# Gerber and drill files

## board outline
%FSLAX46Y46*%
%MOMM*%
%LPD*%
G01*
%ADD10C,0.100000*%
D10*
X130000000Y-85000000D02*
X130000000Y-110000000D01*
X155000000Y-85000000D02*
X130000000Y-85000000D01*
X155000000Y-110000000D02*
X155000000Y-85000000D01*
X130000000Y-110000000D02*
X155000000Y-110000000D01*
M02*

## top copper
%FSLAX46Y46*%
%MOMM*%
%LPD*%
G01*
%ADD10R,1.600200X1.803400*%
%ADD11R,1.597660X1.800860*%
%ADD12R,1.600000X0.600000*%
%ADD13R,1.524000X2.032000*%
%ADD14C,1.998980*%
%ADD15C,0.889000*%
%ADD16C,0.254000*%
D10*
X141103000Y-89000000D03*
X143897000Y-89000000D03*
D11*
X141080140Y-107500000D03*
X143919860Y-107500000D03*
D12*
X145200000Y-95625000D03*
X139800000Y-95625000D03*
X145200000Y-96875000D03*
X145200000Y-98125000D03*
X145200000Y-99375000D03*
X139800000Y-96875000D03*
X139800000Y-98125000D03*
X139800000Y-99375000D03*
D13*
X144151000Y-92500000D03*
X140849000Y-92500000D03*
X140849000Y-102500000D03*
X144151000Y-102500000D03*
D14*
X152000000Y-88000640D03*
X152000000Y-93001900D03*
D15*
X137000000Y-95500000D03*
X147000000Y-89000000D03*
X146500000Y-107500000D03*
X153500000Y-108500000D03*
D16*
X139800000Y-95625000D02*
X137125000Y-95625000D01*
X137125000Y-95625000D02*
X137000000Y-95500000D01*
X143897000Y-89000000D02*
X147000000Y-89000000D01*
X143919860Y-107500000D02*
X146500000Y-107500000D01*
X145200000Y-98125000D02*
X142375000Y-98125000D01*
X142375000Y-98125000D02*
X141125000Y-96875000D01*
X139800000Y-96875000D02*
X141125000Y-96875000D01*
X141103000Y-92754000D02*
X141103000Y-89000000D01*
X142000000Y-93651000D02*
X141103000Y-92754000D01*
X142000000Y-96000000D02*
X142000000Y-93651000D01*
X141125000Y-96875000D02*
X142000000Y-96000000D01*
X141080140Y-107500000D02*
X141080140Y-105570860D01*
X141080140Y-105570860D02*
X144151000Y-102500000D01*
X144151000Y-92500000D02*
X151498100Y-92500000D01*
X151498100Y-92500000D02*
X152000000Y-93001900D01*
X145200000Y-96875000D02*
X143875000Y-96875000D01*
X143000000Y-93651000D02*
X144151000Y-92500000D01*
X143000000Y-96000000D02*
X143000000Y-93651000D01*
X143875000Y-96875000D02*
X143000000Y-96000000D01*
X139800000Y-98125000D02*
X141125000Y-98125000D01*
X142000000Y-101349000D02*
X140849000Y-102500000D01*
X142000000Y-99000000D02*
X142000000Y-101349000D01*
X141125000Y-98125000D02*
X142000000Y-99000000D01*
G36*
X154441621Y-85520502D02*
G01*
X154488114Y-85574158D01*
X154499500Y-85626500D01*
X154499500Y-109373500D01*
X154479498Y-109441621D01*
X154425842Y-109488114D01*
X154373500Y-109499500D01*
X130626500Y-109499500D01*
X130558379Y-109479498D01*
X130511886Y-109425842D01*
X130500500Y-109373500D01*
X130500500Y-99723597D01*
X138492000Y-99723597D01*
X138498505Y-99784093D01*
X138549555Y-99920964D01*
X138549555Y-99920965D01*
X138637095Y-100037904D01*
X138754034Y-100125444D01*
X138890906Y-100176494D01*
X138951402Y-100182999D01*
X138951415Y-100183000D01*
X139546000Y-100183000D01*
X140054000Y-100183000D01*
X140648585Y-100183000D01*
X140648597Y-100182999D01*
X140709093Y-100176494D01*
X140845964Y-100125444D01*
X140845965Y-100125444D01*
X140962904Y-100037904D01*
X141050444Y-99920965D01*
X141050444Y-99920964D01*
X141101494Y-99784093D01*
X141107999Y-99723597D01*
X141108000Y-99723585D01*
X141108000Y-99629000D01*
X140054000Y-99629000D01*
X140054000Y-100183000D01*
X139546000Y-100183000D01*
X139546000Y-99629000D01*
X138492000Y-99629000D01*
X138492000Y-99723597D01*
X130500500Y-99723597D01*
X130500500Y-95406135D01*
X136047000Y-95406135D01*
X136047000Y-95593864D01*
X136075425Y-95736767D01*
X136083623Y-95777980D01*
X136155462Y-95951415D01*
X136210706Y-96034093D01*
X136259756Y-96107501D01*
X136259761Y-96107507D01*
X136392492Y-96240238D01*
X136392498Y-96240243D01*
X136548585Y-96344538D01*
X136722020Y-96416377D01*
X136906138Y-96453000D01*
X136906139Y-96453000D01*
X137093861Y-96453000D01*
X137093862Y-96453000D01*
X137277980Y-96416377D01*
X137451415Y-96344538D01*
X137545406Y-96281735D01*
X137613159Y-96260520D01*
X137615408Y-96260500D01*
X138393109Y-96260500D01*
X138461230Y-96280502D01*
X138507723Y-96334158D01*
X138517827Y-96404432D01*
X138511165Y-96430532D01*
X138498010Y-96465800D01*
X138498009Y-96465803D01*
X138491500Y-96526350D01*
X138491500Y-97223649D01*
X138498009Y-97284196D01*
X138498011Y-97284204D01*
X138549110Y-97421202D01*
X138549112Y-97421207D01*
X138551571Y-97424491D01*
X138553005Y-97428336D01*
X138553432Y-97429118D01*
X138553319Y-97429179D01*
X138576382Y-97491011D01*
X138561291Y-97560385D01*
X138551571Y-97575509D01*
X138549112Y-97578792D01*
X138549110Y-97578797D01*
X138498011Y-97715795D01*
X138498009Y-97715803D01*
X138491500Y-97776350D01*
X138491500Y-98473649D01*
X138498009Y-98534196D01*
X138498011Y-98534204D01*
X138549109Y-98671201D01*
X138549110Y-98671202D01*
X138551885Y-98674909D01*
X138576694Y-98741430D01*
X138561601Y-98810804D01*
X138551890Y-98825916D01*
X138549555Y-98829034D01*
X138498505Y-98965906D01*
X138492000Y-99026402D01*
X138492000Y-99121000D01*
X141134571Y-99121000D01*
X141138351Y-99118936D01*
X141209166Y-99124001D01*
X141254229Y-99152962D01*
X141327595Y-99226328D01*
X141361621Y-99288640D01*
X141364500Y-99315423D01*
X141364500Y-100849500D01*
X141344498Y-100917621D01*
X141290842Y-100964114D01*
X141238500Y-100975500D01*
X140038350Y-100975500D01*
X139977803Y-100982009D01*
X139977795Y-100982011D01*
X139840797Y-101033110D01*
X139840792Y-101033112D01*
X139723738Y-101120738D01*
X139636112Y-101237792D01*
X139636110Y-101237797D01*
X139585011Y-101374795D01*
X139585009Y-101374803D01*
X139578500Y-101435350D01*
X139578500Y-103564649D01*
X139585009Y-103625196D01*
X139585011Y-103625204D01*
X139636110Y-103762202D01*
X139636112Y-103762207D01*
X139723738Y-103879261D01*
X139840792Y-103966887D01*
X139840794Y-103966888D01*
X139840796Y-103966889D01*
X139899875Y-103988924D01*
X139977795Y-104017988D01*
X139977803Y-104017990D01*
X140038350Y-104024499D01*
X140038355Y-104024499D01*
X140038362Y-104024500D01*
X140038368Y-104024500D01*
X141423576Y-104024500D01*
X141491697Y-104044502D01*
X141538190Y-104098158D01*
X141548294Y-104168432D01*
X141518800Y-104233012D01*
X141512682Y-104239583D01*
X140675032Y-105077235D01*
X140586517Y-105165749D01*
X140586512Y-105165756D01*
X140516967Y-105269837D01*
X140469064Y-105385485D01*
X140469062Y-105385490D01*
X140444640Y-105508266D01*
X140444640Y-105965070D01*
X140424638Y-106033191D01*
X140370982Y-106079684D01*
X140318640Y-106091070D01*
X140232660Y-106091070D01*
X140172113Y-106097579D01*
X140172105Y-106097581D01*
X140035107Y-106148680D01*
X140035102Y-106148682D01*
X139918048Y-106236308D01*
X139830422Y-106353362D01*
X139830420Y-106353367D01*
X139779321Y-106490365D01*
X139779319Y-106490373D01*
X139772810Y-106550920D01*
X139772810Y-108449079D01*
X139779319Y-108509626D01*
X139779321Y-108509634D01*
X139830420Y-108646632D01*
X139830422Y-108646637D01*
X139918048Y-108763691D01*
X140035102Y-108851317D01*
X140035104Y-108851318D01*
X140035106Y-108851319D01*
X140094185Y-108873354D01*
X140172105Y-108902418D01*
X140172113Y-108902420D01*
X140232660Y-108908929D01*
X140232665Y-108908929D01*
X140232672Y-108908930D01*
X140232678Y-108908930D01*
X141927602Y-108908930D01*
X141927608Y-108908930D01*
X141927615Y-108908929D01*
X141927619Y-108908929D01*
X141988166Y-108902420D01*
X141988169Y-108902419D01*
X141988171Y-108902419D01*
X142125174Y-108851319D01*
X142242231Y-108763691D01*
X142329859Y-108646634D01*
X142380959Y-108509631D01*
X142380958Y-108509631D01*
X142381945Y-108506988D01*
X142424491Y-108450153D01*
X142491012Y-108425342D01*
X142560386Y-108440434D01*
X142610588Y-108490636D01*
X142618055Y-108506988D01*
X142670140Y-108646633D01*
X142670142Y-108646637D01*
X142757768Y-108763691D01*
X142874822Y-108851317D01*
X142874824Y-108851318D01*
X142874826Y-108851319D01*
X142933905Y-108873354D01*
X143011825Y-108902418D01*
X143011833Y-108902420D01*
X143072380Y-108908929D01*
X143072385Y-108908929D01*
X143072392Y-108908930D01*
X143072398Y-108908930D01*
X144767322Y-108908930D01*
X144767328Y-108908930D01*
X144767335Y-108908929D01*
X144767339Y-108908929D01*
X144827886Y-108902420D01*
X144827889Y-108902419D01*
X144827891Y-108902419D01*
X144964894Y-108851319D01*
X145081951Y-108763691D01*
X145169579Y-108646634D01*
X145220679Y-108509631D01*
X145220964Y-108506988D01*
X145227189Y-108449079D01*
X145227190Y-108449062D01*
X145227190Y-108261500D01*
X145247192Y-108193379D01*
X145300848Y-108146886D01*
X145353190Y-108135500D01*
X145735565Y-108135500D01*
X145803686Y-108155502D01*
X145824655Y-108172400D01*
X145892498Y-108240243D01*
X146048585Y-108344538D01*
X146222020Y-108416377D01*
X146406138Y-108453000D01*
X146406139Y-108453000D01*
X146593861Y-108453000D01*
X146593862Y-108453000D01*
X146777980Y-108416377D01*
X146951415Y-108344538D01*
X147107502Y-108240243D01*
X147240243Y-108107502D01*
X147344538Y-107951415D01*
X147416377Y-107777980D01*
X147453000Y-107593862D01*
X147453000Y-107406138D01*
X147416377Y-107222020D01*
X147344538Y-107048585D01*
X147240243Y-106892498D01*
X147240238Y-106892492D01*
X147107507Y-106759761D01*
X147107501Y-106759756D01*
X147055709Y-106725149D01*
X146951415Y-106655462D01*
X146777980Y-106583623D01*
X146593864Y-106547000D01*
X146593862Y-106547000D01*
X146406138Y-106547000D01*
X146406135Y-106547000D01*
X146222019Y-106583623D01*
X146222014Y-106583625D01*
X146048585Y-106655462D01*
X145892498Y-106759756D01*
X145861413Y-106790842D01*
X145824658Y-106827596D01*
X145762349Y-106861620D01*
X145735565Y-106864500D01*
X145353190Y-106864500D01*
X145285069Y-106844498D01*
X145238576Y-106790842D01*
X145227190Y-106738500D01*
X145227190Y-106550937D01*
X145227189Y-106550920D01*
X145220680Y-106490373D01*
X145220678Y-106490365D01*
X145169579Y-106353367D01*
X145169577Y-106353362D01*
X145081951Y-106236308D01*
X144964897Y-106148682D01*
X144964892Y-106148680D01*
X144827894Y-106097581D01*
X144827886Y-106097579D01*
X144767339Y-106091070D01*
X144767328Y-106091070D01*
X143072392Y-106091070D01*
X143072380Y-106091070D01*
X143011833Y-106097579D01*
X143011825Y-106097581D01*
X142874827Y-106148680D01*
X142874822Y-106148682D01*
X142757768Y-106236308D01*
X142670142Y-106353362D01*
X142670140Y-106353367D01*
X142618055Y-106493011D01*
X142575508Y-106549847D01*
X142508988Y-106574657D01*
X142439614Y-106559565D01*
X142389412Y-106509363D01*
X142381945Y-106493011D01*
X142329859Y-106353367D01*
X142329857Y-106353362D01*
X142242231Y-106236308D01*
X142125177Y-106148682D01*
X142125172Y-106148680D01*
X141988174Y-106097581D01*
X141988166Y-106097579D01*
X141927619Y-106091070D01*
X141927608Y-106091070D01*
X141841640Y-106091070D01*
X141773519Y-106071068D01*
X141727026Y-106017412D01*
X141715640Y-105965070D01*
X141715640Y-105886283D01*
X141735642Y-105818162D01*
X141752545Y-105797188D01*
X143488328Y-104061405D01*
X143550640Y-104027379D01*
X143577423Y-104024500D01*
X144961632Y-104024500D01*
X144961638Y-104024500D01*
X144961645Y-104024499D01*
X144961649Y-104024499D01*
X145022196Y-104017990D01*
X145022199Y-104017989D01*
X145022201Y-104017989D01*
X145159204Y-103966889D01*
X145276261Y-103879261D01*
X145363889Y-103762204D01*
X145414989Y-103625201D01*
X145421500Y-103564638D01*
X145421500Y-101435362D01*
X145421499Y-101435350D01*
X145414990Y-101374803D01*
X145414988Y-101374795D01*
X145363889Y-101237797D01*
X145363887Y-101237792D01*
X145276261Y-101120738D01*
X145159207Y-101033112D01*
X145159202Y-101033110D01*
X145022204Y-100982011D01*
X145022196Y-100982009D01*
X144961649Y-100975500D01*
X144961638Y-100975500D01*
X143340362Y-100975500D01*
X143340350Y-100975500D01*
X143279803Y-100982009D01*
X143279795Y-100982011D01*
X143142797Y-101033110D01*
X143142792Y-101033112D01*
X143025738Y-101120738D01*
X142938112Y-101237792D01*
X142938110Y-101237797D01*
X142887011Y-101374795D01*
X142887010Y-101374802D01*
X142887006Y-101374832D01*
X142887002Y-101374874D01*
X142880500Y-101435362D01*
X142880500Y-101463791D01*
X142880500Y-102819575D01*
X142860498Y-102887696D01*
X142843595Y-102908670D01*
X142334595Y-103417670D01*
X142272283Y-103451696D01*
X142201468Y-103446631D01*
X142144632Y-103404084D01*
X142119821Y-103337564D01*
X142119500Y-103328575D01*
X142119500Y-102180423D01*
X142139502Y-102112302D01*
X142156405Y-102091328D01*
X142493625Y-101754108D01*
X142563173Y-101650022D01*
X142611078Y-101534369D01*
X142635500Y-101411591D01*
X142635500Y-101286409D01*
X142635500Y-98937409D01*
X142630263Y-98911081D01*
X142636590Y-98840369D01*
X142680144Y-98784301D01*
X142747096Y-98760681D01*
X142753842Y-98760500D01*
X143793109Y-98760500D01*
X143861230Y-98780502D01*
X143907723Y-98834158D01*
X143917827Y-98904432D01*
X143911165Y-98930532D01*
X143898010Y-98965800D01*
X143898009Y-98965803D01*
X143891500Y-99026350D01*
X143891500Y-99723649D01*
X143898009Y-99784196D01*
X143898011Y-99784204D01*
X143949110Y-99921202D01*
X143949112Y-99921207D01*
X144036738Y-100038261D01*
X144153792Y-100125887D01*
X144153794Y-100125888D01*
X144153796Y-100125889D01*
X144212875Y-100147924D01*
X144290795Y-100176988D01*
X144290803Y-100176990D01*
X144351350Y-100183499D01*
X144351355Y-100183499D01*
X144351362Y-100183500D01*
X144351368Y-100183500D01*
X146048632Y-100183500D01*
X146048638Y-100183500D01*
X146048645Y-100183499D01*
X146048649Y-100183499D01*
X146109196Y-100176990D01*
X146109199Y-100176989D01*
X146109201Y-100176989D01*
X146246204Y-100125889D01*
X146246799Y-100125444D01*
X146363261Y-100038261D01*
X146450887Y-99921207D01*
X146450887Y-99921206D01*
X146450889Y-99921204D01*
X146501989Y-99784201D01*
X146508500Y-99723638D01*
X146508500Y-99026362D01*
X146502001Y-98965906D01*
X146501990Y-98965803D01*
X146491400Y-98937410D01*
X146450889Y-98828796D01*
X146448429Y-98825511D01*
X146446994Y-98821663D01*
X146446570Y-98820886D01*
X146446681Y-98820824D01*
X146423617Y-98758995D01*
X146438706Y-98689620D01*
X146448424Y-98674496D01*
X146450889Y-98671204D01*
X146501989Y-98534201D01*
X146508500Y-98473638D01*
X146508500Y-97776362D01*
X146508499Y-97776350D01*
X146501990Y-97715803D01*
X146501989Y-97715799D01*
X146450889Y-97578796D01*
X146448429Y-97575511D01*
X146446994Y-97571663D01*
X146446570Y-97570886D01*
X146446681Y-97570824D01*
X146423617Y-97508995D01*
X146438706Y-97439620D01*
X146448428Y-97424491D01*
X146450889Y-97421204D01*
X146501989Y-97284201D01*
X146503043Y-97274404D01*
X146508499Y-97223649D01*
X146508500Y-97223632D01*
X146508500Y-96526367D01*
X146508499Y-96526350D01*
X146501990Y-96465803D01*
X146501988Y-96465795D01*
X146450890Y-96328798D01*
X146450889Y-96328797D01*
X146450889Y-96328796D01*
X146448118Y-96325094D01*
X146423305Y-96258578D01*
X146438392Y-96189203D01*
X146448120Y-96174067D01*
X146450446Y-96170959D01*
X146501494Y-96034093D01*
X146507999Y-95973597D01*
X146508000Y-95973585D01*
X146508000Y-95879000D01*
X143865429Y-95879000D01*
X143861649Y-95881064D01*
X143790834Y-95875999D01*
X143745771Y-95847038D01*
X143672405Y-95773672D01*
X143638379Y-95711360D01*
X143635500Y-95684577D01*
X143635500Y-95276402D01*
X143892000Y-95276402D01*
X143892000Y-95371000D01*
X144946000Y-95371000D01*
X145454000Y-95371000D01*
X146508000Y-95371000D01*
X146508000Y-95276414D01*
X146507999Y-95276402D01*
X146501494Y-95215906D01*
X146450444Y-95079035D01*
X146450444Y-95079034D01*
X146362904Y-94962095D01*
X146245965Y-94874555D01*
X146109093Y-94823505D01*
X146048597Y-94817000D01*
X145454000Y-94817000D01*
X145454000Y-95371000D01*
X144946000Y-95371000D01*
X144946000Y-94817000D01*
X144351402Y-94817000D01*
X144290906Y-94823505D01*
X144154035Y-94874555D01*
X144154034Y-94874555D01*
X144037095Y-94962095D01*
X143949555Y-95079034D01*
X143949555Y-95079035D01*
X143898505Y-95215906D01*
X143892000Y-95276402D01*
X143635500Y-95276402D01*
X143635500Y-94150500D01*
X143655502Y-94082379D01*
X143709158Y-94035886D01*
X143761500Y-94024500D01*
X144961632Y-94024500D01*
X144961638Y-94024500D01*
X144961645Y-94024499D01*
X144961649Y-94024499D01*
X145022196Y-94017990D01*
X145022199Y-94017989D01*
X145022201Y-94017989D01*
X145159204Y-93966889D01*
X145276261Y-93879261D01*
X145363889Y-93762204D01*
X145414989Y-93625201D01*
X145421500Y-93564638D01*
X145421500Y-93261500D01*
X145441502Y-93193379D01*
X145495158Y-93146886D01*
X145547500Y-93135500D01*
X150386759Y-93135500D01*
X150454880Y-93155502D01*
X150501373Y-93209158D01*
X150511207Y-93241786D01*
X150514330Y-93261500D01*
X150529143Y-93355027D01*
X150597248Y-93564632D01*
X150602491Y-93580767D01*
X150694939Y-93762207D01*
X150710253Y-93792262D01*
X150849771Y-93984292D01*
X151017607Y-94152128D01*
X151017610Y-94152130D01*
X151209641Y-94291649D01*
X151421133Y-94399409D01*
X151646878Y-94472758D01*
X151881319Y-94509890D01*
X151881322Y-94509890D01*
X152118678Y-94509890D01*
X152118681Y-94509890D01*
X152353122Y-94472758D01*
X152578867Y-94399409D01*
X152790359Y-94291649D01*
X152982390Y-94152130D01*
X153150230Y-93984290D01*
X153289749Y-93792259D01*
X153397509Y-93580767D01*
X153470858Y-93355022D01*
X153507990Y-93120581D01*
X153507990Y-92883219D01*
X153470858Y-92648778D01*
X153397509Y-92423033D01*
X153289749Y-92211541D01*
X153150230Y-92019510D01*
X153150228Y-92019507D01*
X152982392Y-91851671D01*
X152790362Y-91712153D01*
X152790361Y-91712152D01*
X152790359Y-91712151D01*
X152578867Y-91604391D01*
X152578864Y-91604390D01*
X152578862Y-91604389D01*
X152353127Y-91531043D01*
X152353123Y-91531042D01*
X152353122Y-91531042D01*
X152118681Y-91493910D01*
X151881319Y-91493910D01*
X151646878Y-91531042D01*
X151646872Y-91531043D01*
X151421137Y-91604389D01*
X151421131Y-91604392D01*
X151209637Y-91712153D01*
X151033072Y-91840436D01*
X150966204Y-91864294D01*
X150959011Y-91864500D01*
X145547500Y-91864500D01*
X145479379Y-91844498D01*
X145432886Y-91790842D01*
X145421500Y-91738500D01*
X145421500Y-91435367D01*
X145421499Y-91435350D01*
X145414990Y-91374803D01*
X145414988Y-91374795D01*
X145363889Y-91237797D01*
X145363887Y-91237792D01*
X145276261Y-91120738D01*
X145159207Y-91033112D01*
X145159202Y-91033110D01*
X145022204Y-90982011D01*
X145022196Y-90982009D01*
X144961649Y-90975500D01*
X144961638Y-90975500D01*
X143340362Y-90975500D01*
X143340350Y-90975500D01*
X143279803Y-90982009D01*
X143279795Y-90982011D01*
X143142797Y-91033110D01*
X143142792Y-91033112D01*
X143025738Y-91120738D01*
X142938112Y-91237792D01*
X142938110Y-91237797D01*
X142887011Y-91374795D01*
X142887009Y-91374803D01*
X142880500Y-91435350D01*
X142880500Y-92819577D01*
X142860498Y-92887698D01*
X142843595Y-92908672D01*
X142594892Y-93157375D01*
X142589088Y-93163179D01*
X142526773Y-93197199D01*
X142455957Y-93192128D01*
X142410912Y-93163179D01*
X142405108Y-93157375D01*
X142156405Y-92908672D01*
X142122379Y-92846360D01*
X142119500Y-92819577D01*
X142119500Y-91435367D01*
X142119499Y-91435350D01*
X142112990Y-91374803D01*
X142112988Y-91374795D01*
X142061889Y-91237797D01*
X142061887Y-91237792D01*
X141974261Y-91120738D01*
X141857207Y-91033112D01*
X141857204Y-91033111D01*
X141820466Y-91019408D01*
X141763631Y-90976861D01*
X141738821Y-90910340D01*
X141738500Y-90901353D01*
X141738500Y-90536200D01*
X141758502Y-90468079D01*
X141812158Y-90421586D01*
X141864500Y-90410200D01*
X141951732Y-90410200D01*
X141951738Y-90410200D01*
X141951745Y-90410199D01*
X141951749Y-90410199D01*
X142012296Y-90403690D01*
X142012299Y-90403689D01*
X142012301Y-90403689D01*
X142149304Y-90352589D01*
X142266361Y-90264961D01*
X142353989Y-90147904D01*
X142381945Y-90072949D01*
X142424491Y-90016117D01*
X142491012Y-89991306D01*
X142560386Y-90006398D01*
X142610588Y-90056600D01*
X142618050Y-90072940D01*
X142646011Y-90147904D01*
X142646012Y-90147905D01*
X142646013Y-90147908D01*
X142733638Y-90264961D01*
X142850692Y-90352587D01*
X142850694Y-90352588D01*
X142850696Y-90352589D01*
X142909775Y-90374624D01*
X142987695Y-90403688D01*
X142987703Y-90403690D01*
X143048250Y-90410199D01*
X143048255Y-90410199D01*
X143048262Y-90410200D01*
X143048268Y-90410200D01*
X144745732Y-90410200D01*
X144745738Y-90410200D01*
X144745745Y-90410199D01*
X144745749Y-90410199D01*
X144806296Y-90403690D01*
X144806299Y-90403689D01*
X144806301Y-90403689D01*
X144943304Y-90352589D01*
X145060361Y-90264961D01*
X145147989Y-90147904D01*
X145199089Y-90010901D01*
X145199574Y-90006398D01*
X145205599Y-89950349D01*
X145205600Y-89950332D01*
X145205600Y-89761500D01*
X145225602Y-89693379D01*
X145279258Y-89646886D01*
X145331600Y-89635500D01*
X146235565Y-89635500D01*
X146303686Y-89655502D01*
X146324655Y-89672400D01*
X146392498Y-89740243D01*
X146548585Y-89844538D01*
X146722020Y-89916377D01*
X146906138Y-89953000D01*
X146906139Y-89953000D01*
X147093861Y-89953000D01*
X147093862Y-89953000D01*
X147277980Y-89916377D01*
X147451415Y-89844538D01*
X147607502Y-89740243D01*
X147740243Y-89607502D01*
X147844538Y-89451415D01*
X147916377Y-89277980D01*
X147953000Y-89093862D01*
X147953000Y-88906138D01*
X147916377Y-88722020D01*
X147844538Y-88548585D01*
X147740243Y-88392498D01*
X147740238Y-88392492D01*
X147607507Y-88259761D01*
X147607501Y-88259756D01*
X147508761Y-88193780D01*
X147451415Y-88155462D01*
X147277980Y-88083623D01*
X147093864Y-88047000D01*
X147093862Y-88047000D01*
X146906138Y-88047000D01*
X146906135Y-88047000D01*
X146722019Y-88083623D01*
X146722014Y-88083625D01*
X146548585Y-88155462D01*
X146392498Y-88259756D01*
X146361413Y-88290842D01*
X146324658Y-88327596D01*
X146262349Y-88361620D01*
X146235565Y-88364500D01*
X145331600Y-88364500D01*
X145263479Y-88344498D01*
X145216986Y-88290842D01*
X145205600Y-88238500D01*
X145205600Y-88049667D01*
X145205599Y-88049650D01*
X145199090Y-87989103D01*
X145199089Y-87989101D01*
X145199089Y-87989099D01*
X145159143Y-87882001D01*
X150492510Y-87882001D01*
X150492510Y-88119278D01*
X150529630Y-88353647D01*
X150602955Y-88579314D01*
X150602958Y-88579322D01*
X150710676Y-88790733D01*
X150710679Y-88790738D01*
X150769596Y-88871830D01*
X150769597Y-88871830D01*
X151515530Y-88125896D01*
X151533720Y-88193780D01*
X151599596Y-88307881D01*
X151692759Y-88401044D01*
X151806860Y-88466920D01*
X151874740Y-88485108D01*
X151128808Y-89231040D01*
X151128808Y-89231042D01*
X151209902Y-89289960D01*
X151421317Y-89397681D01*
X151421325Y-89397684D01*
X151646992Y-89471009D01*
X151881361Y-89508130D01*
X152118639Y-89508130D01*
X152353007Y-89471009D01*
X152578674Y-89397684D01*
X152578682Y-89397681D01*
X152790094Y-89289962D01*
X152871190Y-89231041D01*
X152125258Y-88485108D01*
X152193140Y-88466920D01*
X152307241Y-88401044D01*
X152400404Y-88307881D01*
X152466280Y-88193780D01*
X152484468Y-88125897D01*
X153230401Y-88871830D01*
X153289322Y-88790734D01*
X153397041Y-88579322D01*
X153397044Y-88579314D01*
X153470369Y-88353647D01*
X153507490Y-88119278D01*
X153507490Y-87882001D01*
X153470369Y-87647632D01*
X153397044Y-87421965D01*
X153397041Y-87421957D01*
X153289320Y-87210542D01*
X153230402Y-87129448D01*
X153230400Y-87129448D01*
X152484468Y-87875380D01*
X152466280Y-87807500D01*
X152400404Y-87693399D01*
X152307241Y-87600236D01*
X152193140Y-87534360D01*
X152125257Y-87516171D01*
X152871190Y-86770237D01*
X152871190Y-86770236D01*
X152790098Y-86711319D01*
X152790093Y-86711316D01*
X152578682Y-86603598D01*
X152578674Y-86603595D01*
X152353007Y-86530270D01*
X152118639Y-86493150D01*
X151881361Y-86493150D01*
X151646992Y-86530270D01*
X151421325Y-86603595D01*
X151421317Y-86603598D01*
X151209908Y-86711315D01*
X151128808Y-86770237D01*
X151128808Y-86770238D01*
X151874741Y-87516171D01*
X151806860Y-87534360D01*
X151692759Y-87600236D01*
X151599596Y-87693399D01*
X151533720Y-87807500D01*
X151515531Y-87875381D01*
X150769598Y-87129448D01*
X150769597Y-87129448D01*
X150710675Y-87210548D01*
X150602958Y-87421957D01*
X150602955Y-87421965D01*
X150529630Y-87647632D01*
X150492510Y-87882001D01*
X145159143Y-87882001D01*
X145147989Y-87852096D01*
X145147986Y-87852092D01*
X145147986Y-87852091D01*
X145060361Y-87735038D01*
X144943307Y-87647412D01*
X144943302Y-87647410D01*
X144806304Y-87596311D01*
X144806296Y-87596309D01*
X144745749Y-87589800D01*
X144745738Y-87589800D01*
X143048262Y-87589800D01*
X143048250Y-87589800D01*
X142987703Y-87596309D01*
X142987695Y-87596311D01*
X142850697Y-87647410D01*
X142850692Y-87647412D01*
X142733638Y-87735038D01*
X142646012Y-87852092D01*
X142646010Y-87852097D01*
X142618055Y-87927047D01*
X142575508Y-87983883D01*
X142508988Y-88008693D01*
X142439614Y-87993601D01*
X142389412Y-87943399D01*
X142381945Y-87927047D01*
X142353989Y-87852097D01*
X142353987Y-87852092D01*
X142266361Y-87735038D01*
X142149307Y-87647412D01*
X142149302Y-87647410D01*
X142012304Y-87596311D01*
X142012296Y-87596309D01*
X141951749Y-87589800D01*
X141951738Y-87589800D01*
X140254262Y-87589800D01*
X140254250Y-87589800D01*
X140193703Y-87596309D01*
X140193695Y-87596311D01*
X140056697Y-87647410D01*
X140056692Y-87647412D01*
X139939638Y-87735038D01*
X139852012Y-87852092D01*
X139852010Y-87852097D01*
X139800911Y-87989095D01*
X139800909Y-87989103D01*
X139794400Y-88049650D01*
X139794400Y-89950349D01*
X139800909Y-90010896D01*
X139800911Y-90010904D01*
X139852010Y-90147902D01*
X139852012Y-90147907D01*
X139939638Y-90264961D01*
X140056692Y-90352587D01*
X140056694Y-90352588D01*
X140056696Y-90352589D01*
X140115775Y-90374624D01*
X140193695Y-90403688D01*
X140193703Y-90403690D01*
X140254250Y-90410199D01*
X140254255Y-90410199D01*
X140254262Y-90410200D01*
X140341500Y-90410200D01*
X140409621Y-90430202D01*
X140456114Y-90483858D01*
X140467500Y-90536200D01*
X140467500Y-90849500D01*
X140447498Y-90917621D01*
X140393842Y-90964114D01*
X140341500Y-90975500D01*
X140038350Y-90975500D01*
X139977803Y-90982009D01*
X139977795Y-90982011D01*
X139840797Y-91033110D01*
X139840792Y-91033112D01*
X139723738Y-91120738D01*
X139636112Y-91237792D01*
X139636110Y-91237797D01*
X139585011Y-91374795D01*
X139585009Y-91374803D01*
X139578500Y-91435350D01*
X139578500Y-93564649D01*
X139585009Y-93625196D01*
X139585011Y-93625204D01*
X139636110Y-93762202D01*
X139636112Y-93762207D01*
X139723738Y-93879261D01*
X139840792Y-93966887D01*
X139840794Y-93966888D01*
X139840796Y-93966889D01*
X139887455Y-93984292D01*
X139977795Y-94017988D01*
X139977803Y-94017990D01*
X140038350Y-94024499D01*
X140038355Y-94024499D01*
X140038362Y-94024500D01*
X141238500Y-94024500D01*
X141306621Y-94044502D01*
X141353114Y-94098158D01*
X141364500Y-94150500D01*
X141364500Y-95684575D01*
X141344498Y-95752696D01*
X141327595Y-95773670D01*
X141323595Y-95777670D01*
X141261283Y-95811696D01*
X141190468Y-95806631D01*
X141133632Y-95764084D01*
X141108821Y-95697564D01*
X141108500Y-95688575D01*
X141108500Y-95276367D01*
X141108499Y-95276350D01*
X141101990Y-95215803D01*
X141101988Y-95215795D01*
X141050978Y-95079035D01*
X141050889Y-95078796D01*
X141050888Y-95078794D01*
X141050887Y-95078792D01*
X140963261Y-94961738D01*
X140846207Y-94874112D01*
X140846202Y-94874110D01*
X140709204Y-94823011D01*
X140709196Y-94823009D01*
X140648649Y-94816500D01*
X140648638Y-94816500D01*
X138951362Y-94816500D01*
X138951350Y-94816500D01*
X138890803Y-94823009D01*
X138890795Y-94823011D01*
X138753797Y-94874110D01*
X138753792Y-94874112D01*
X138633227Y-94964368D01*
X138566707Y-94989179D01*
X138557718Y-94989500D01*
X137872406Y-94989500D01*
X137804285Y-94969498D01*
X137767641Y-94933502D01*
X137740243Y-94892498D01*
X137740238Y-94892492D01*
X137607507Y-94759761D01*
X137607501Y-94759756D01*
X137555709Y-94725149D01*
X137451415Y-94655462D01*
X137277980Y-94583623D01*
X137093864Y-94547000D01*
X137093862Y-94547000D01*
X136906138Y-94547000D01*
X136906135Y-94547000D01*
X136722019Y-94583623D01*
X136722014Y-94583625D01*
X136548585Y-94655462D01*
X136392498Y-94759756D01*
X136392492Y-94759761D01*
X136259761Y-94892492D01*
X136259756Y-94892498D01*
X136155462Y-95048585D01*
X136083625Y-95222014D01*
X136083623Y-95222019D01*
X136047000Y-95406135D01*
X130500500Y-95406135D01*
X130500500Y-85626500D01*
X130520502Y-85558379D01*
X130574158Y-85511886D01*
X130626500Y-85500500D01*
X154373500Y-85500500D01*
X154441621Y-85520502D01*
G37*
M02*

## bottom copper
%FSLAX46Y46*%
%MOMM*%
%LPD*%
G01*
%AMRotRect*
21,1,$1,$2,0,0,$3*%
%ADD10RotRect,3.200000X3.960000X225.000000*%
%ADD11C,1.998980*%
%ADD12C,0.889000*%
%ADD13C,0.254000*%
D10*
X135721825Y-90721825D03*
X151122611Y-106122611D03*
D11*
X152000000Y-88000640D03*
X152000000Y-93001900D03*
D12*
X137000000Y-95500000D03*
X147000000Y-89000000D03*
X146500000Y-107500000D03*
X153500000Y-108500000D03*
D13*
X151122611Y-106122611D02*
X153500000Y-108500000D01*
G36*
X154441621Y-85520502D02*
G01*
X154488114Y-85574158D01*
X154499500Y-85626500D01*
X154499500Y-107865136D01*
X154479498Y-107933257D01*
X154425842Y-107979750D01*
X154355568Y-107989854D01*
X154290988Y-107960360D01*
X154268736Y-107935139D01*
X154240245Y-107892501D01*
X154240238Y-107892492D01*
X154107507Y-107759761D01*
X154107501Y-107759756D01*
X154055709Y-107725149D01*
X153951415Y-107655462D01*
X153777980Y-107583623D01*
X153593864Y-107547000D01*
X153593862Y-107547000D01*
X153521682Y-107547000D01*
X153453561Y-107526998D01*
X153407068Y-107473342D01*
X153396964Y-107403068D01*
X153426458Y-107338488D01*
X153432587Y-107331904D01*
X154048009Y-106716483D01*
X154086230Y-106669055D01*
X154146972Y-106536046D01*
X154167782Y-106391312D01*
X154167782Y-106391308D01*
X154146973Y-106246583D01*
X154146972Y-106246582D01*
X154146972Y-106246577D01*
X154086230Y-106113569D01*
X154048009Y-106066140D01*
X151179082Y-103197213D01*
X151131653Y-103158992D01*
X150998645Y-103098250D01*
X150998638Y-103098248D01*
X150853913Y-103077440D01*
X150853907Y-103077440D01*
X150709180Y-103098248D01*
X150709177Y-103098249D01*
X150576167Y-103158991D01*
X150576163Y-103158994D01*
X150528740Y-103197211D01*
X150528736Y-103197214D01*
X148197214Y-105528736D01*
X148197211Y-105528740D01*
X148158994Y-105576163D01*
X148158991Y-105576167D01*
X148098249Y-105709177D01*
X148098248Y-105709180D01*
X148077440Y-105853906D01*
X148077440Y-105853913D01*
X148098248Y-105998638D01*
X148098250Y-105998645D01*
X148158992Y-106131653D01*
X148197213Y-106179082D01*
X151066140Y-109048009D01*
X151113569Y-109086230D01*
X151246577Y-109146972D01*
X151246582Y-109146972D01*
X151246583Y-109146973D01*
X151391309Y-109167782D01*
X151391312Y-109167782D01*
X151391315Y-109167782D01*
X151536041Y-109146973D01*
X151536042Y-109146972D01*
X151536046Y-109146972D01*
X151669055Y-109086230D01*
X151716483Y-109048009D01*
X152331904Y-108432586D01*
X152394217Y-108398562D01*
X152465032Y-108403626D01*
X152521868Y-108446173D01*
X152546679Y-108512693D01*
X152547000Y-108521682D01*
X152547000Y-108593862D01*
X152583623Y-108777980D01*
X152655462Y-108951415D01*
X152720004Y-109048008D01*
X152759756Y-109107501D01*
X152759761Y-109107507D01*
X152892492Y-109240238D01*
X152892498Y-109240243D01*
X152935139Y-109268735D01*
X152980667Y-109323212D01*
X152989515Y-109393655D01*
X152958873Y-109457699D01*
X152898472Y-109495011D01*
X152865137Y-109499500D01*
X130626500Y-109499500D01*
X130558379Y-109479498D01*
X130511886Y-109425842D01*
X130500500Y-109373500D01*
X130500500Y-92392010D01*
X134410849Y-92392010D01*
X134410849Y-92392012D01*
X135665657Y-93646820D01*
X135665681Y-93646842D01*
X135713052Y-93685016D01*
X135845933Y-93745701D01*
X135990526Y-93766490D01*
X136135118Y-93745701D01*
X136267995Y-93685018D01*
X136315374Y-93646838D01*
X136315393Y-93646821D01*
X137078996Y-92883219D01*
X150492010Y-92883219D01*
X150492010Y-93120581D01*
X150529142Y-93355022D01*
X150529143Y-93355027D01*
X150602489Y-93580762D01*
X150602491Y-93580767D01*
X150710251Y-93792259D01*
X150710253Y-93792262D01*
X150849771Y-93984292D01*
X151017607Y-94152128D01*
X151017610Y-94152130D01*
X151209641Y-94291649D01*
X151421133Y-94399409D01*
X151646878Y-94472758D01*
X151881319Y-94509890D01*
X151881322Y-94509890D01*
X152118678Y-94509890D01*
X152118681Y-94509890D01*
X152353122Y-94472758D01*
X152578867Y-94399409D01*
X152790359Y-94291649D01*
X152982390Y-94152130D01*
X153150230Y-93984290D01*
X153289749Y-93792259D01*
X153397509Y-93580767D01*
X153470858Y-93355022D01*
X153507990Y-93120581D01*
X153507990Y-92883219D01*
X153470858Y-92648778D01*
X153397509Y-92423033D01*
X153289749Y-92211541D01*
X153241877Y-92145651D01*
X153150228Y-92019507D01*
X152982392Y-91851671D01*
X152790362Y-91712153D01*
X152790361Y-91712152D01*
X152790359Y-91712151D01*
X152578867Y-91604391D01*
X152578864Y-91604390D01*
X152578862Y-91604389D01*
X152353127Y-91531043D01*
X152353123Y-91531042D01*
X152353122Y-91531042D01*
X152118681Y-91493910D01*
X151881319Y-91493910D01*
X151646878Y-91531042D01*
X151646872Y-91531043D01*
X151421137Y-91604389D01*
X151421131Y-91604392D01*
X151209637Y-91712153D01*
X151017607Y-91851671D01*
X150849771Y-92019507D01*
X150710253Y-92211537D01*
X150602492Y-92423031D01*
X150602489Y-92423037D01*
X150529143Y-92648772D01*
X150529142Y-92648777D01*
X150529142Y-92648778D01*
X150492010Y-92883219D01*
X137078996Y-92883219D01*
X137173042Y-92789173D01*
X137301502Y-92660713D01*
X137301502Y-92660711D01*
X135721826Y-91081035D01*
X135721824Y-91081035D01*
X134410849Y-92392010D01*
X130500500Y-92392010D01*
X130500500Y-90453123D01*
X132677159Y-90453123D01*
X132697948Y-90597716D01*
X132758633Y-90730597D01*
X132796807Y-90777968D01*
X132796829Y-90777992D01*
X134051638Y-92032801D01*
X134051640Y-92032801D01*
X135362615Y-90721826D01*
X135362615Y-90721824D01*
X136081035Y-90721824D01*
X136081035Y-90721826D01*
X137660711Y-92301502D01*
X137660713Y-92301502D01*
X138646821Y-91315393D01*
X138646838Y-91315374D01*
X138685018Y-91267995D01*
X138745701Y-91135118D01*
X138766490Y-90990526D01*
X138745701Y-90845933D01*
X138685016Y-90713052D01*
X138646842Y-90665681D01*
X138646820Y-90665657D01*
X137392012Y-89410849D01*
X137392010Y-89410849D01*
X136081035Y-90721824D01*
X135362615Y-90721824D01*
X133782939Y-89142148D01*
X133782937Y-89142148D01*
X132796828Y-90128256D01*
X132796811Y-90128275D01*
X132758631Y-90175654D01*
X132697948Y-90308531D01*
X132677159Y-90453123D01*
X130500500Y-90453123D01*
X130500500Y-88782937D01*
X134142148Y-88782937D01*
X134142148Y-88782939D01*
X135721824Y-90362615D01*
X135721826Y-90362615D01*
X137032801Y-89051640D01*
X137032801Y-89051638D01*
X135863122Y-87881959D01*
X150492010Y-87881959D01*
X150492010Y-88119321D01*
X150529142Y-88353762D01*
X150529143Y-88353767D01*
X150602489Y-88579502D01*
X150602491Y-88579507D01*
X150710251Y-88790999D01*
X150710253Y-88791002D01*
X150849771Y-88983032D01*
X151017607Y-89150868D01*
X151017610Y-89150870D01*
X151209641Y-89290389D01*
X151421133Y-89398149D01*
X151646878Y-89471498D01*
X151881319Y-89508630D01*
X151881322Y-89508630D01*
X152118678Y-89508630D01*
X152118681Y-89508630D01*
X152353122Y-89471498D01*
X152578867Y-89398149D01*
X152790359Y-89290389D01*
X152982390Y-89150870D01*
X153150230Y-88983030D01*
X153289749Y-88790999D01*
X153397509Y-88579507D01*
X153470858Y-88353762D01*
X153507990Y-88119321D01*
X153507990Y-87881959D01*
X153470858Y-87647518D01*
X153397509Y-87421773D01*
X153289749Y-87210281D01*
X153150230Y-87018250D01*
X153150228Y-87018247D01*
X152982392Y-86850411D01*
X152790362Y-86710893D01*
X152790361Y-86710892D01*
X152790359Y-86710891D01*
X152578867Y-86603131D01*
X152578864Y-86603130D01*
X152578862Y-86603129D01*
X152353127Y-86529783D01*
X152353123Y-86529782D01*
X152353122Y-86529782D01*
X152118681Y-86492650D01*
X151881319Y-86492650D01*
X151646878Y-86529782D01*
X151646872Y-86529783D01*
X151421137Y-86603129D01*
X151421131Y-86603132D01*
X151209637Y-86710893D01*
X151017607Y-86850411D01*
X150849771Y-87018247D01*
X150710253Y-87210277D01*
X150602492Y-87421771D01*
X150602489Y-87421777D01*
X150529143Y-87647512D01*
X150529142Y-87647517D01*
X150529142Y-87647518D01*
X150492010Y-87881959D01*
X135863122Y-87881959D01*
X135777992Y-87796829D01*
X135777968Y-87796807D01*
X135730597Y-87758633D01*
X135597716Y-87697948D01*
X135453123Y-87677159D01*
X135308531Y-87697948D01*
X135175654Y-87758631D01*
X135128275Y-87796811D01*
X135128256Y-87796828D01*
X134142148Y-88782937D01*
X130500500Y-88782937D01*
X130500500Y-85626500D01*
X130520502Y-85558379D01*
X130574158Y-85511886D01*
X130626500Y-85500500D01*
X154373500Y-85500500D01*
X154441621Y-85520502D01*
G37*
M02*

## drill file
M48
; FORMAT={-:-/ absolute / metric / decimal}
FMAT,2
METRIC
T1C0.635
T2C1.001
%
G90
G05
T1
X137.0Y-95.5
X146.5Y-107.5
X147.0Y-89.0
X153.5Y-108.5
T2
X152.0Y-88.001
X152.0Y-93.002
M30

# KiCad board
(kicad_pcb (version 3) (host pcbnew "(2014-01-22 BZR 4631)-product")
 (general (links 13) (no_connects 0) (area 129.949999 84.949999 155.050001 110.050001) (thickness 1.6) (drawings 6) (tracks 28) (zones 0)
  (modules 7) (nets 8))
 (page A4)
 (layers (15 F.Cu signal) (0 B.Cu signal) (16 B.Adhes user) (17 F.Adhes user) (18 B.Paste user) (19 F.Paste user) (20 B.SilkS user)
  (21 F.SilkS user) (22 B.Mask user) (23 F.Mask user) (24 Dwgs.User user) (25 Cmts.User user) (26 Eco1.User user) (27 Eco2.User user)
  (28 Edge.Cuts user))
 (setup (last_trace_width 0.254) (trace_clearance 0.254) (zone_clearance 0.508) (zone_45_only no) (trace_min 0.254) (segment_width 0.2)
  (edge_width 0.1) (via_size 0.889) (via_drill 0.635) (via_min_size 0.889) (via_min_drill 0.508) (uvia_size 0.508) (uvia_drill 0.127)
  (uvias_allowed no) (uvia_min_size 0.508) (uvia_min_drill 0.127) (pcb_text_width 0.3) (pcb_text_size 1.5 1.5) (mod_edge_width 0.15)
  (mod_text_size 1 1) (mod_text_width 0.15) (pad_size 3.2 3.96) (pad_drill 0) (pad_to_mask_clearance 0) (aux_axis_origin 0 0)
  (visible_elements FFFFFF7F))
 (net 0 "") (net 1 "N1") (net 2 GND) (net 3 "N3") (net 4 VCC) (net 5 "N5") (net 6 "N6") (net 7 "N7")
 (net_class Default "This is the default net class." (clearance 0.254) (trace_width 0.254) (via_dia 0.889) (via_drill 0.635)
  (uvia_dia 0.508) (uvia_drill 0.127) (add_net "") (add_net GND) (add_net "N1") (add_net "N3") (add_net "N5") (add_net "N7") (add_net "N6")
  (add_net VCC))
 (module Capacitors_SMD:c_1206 (layer F.Cu) (at 142.5 89 180)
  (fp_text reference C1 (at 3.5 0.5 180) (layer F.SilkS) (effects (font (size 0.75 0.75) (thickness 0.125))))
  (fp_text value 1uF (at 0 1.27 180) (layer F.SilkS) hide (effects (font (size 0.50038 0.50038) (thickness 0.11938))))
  (pad 1 smd rect (at 1.397 0 180) (size 1.6002 1.8034) (layers F.Cu F.Paste F.Mask) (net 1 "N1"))
  (pad 2 smd rect (at -1.397 0 180) (size 1.6002 1.8034) (layers F.Cu F.Paste F.Mask) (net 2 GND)))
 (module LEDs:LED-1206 (layer F.Cu) (at 142.5 107.5)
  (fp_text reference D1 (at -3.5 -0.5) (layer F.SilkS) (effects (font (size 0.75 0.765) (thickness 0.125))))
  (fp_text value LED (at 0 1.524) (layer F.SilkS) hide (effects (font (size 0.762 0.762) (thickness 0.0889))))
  (pad 1 smd rect (at -1.41986 0) (size 1.59766 1.80086) (layers F.Cu F.Paste F.Mask) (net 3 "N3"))
  (pad 2 smd rect (at 1.41986 0) (size 1.59766 1.80086) (layers F.Cu F.Paste F.Mask) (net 2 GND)))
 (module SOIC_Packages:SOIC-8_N (layer F.Cu) (at 142.5 97.5 270)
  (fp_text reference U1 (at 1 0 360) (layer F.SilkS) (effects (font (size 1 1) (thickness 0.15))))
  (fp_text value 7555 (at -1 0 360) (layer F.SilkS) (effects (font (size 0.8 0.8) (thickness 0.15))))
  (pad 8 smd rect (at -1.875 -2.7 270) (size 0.6 1.6) (layers F.Cu F.Paste F.Mask) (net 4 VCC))
  (pad 1 smd rect (at -1.875 2.7 270) (size 0.6 1.6) (layers F.Cu F.Paste F.Mask) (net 2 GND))
  (pad 7 smd rect (at -0.625 -2.7 270) (size 0.6 1.6) (layers F.Cu F.Paste F.Mask) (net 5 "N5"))
  (pad 6 smd rect (at 0.625 -2.7 270) (size 0.6 1.6) (layers F.Cu F.Paste F.Mask) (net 1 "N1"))
  (pad 5 smd rect (at 1.875 -2.7 270) (size 0.6 1.6) (layers F.Cu F.Paste F.Mask) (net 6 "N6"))
  (pad 2 smd rect (at -0.625 2.7 270) (size 0.6 1.6) (layers F.Cu F.Paste F.Mask) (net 1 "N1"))
  (pad 3 smd rect (at 0.625 2.7 270) (size 0.6 1.6) (layers F.Cu F.Paste F.Mask) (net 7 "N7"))
  (pad 4 smd rect (at 1.875 2.7 270) (size 0.6 1.6) (layers F.Cu F.Paste F.Mask) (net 4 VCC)))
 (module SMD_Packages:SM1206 (layer F.Cu) (at 142.5 92.5 180)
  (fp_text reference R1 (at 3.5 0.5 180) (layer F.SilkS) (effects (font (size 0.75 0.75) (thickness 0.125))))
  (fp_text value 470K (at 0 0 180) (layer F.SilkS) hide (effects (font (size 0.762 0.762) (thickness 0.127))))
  (pad 1 smd rect (at -1.651 0 180) (size 1.524 2.032) (layers F.Cu F.Paste F.Mask) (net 5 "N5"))
  (pad 2 smd rect (at 1.651 0 180) (size 1.524 2.032) (layers F.Cu F.Paste F.Mask) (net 1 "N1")))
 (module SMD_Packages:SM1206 (layer F.Cu) (at 142.5 102.5)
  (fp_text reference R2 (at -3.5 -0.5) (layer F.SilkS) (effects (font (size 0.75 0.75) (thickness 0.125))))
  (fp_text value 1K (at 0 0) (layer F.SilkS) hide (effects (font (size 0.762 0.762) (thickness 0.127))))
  (pad 1 smd rect (at -1.651 0) (size 1.524 2.032) (layers F.Cu F.Paste F.Mask) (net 7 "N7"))
  (pad 2 smd rect (at 1.651 0) (size 1.524 2.032) (layers F.Cu F.Paste F.Mask) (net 3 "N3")))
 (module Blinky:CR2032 (layer B.Cu) (at 143.5 98.5 225)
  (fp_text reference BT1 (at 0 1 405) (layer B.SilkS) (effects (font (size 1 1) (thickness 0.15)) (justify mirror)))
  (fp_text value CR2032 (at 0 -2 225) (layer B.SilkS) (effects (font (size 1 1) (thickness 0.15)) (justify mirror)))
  (pad 2 smd rect (at 0 11 225) (size 3.2 3.96) (layers B.Cu B.Paste B.Mask) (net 2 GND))
  (pad 1 smd rect (at 0 -10.78 225) (size 3.2 3.96) (layers B.Cu B.Paste B.Mask) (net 4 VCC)))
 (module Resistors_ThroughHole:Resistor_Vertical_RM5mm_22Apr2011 (layer F.Cu) (at 152 90.5 270)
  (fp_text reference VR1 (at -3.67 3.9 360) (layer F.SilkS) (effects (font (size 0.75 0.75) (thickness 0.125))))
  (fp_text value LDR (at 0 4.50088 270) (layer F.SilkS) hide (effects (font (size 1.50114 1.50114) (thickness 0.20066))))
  (pad 1 thru_hole circle (at -2.49936 0 270) (size 1.99898 1.99898) (drill 1.00076) (layers *.Cu) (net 4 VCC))
  (pad 2 thru_hole circle (at 2.5019 0 270) (size 1.99898 1.99898) (drill 1.00076) (layers *.Cu) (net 5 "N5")))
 (gr_line (start 130 85) (end 130 110) (angle 90) (layer Edge.Cuts) (width 0.1))
 (gr_line (start 155 85) (end 130 85) (angle 90) (layer Edge.Cuts) (width 0.1))
 (gr_line (start 155 110) (end 155 85) (angle 90) (layer Edge.Cuts) (width 0.1))
 (gr_line (start 130 110) (end 155 110) (angle 90) (layer Edge.Cuts) (width 0.1))
 (segment (start 139.8 95.625) (end 137.125 95.625) (width 0.254) (layer F.Cu) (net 2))
 (via (at 137 95.5) (size 0.889) (layers F.Cu B.Cu) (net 2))
 (segment (start 137.125 95.625) (end 137 95.5) (width 0.254) (layer F.Cu) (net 2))
 (segment (start 143.897 89) (end 147 89) (width 0.254) (layer F.Cu) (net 2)) (via (at 147 89) (size 0.889) (layers F.Cu B.Cu) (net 2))
 (segment (start 143.91986 107.5) (end 146.5 107.5) (width 0.254) (layer F.Cu) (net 2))
 (via (at 146.5 107.5) (size 0.889) (layers F.Cu B.Cu) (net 2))
 (segment (start 145.2 98.125) (end 142.375 98.125) (width 0.254) (layer F.Cu) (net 1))
 (segment (start 142.375 98.125) (end 141.125 96.875) (width 0.254) (layer F.Cu) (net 1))
 (segment (start 139.8 96.875) (end 141.125 96.875) (width 0.254) (layer F.Cu) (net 1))
 (segment (start 141.103 92.754) (end 141.103 89) (width 0.254) (layer F.Cu) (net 1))
 (segment (start 142 93.651) (end 141.103 92.754) (width 0.254) (layer F.Cu) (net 1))
 (segment (start 142 96) (end 142 93.651) (width 0.254) (layer F.Cu) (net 1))
 (segment (start 141.125 96.875) (end 142 96) (width 0.254) (layer F.Cu) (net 1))
 (segment (start 141.08014 107.5) (end 141.08014 105.57086) (width 0.254) (layer F.Cu) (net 3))
 (segment (start 141.08014 105.57086) (end 144.151 102.5) (width 0.254) (layer F.Cu) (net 3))
 (segment (start 144.151 92.5) (end 151.4981 92.5) (width 0.254) (layer F.Cu) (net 5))
 (segment (start 151.4981 92.5) (end 152 93.0019) (width 0.254) (layer F.Cu) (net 5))
 (segment (start 145.2 96.875) (end 143.875 96.875) (width 0.254) (layer F.Cu) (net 5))
 (segment (start 143 93.651) (end 144.151 92.5) (width 0.254) (layer F.Cu) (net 5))
 (segment (start 143 96) (end 143 93.651) (width 0.254) (layer F.Cu) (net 5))
 (segment (start 143.875 96.875) (end 143 96) (width 0.254) (layer F.Cu) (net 5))
 (segment (start 139.8 98.125) (end 141.125 98.125) (width 0.254) (layer F.Cu) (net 7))
 (segment (start 142 101.349) (end 140.849 102.5) (width 0.254) (layer F.Cu) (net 7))
 (segment (start 142 99) (end 142 101.349) (width 0.254) (layer F.Cu) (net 7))
 (segment (start 141.125 98.125) (end 142 99) (width 0.254) (layer F.Cu) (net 7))
 (segment (start 151.122611 106.122611) (end 153.5 108.5) (width 0.254) (layer B.Cu) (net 4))
 (via (at 153.5 108.5) (size 0.889) (layers F.Cu B.Cu) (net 4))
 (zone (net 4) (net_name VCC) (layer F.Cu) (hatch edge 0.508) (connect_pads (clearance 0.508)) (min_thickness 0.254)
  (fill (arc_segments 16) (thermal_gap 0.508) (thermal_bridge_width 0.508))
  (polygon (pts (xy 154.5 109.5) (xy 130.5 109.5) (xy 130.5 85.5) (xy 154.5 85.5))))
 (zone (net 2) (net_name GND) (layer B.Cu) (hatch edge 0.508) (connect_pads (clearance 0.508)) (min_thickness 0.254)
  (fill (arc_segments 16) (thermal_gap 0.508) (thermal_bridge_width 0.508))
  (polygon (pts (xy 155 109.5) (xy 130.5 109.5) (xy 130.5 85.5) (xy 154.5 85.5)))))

